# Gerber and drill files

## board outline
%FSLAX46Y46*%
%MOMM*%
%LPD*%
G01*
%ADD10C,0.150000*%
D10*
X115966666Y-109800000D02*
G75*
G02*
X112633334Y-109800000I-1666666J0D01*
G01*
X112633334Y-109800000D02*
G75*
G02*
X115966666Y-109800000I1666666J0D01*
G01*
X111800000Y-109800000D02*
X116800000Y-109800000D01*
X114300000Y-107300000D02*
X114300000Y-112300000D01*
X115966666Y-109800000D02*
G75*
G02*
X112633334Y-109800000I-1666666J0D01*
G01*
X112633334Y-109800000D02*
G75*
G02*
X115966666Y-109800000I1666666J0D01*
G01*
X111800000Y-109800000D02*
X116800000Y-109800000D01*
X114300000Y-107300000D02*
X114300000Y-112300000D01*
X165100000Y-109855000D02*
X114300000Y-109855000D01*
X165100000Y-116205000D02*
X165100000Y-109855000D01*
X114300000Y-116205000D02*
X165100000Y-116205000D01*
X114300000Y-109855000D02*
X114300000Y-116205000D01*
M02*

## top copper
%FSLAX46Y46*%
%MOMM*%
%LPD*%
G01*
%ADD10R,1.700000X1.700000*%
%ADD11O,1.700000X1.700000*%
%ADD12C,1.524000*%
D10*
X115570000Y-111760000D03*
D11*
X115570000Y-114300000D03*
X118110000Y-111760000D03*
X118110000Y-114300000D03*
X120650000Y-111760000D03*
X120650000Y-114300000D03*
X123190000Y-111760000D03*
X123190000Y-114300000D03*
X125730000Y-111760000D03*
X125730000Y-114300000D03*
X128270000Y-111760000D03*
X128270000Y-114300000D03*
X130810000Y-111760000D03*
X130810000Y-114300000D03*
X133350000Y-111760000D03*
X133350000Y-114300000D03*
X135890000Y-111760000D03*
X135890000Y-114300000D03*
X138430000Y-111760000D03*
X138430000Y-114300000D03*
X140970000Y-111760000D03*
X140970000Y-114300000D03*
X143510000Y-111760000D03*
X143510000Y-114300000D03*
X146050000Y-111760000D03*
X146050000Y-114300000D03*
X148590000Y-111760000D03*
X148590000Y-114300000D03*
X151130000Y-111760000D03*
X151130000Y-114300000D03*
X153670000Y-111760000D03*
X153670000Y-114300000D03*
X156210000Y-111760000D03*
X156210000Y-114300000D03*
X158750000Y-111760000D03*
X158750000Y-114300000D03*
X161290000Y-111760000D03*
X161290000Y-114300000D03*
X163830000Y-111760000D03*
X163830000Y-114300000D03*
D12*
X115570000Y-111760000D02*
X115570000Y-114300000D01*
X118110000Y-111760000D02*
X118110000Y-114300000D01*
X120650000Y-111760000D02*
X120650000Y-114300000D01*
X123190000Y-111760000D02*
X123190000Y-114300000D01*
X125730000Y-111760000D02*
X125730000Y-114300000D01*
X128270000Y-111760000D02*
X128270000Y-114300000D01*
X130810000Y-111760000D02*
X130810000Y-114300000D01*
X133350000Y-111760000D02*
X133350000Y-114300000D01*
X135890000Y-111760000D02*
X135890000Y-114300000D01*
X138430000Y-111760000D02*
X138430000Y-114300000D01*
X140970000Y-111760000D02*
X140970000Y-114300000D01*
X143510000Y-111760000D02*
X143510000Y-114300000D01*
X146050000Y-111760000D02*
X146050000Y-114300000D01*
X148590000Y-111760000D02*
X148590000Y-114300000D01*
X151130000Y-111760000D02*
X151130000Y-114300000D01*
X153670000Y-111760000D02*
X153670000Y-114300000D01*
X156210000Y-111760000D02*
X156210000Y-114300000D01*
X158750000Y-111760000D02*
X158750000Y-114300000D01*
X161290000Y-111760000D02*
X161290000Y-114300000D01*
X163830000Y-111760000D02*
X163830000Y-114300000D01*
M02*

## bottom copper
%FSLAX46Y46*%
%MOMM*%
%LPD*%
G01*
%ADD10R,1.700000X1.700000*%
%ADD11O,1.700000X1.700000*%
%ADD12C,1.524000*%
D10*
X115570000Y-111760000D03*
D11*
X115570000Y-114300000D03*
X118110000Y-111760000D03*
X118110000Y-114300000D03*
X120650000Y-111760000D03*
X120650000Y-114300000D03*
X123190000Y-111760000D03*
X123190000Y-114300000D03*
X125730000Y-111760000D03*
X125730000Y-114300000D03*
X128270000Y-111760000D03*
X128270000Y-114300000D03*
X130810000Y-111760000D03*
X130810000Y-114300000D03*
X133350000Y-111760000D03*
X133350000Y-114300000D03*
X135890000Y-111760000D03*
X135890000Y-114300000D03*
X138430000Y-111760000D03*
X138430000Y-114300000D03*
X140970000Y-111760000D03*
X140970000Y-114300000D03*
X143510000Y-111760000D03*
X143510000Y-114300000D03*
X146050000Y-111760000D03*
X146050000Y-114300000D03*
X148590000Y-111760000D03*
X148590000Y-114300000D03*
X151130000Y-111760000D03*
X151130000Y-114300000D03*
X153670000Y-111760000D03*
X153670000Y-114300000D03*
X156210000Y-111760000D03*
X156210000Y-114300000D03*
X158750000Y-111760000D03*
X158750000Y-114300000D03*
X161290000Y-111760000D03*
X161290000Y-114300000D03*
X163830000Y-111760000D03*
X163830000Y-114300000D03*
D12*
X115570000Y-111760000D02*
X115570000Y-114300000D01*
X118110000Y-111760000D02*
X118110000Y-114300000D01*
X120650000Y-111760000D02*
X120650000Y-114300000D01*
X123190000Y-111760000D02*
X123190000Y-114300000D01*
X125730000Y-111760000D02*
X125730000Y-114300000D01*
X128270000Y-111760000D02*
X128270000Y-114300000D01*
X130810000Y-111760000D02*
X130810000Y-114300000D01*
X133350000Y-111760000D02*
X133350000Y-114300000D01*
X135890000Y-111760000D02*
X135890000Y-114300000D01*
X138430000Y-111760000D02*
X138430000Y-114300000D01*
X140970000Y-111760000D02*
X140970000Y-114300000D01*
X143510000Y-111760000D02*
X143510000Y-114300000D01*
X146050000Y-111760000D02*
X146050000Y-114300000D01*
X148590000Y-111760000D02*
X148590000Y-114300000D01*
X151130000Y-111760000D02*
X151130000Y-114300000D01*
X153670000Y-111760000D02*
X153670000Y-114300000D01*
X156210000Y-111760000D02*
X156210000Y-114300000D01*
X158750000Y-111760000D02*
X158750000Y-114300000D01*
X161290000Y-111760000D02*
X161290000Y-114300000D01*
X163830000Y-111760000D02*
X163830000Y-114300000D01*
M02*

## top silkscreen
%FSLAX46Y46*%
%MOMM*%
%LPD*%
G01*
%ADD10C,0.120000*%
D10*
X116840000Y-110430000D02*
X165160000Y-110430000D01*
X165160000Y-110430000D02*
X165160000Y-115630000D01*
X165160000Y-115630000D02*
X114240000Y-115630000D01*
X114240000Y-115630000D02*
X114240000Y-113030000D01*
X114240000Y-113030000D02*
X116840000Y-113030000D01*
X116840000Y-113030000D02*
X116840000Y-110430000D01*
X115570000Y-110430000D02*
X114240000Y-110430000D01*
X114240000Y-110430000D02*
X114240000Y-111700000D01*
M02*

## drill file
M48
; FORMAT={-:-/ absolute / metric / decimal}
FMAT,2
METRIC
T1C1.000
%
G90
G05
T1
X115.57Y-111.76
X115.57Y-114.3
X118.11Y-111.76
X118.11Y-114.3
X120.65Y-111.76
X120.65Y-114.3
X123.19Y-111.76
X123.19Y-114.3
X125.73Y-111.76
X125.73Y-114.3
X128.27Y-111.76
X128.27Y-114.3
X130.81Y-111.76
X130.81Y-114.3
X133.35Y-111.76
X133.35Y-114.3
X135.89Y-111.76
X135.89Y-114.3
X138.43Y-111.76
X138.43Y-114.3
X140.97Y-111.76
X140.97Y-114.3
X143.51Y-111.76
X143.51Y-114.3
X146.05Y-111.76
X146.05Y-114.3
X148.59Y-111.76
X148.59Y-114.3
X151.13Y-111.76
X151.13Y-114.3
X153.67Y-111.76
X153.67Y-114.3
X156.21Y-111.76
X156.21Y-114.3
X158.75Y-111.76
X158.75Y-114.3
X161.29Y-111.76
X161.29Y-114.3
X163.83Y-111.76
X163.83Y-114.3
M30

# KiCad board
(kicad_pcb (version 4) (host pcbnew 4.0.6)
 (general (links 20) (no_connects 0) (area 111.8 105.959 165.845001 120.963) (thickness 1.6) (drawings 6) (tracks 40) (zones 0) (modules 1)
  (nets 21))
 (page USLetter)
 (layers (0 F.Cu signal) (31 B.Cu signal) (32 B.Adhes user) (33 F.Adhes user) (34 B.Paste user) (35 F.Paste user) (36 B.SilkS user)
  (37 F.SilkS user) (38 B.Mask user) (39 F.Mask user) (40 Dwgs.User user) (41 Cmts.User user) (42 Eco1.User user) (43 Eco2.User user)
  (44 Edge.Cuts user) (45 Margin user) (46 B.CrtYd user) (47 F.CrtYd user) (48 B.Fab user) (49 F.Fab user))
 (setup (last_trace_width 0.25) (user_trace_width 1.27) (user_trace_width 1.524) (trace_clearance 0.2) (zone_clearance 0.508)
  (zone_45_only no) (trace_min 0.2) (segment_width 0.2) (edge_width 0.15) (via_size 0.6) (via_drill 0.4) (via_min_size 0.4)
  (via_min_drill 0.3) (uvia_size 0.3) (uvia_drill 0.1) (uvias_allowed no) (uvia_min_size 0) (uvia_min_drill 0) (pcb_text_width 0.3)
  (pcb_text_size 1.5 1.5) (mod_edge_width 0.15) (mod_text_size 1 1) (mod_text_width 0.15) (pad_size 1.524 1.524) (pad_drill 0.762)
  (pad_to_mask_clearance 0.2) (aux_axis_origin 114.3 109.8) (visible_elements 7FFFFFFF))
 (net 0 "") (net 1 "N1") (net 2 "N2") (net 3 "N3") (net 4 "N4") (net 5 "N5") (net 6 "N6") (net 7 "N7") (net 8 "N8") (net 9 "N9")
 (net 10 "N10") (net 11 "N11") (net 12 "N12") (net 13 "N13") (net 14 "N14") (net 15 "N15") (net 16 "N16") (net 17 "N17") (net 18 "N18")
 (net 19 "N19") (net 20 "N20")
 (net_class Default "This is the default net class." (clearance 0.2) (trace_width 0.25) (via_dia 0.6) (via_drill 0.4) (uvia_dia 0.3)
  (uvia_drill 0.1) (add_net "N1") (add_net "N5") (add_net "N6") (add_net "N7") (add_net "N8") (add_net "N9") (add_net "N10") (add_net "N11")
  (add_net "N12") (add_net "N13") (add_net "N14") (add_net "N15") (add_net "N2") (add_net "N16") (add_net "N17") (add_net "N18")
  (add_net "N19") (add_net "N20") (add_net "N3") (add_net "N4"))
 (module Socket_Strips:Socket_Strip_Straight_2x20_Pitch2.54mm (layer F.Cu) (at 115.57 111.76 90)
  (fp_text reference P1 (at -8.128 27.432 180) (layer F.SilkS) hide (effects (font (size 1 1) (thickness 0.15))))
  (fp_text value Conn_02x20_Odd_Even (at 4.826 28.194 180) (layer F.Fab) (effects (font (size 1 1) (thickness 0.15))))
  (fp_line (start 1.33 1.27) (end 1.33 49.59) (layer F.SilkS) (width 0.12))
  (fp_line (start 1.33 49.59) (end -3.87 49.59) (layer F.SilkS) (width 0.12))
  (fp_line (start -3.87 49.59) (end -3.87 -1.33) (layer F.SilkS) (width 0.12))
  (fp_line (start -3.87 -1.33) (end -1.27 -1.33) (layer F.SilkS) (width 0.12))
  (fp_line (start -1.27 -1.33) (end -1.27 1.27) (layer F.SilkS) (width 0.12))
  (fp_line (start -1.27 1.27) (end 1.33 1.27) (layer F.SilkS) (width 0.12))
  (fp_line (start 1.33 0) (end 1.33 -1.33) (layer F.SilkS) (width 0.12))
  (fp_line (start 1.33 -1.33) (end 0.06 -1.33) (layer F.SilkS) (width 0.12))
  (pad 1 thru_hole rect (at 0 0 90) (size 1.7 1.7) (drill 1) (layers *.Cu *.Mask) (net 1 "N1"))
  (pad 2 thru_hole oval (at -2.54 0 90) (size 1.7 1.7) (drill 1) (layers *.Cu *.Mask) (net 1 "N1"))
  (pad 3 thru_hole oval (at 0 2.54 90) (size 1.7 1.7) (drill 1) (layers *.Cu *.Mask) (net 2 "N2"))
  (pad 4 thru_hole oval (at -2.54 2.54 90) (size 1.7 1.7) (drill 1) (layers *.Cu *.Mask) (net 2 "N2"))
  (pad 5 thru_hole oval (at 0 5.08 90) (size 1.7 1.7) (drill 1) (layers *.Cu *.Mask) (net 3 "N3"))
  (pad 6 thru_hole oval (at -2.54 5.08 90) (size 1.7 1.7) (drill 1) (layers *.Cu *.Mask) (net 3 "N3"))
  (pad 7 thru_hole oval (at 0 7.62 90) (size 1.7 1.7) (drill 1) (layers *.Cu *.Mask) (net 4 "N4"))
  (pad 8 thru_hole oval (at -2.54 7.62 90) (size 1.7 1.7) (drill 1) (layers *.Cu *.Mask) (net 4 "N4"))
  (pad 9 thru_hole oval (at 0 10.16 90) (size 1.7 1.7) (drill 1) (layers *.Cu *.Mask) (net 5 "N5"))
  (pad 10 thru_hole oval (at -2.54 10.16 90) (size 1.7 1.7) (drill 1) (layers *.Cu *.Mask) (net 5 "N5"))
  (pad 11 thru_hole oval (at 0 12.7 90) (size 1.7 1.7) (drill 1) (layers *.Cu *.Mask) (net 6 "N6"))
  (pad 12 thru_hole oval (at -2.54 12.7 90) (size 1.7 1.7) (drill 1) (layers *.Cu *.Mask) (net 6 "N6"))
  (pad 13 thru_hole oval (at 0 15.24 90) (size 1.7 1.7) (drill 1) (layers *.Cu *.Mask) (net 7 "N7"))
  (pad 14 thru_hole oval (at -2.54 15.24 90) (size 1.7 1.7) (drill 1) (layers *.Cu *.Mask) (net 7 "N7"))
  (pad 15 thru_hole oval (at 0 17.78 90) (size 1.7 1.7) (drill 1) (layers *.Cu *.Mask) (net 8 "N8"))
  (pad 16 thru_hole oval (at -2.54 17.78 90) (size 1.7 1.7) (drill 1) (layers *.Cu *.Mask) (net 8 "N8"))
  (pad 17 thru_hole oval (at 0 20.32 90) (size 1.7 1.7) (drill 1) (layers *.Cu *.Mask) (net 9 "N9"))
  (pad 18 thru_hole oval (at -2.54 20.32 90) (size 1.7 1.7) (drill 1) (layers *.Cu *.Mask) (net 9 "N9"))
  (pad 19 thru_hole oval (at 0 22.86 90) (size 1.7 1.7) (drill 1) (layers *.Cu *.Mask) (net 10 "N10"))
  (pad 20 thru_hole oval (at -2.54 22.86 90) (size 1.7 1.7) (drill 1) (layers *.Cu *.Mask) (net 10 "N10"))
  (pad 21 thru_hole oval (at 0 25.4 90) (size 1.7 1.7) (drill 1) (layers *.Cu *.Mask) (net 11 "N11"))
  (pad 22 thru_hole oval (at -2.54 25.4 90) (size 1.7 1.7) (drill 1) (layers *.Cu *.Mask) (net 11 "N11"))
  (pad 23 thru_hole oval (at 0 27.94 90) (size 1.7 1.7) (drill 1) (layers *.Cu *.Mask) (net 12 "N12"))
  (pad 24 thru_hole oval (at -2.54 27.94 90) (size 1.7 1.7) (drill 1) (layers *.Cu *.Mask) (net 12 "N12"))
  (pad 25 thru_hole oval (at 0 30.48 90) (size 1.7 1.7) (drill 1) (layers *.Cu *.Mask) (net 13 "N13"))
  (pad 26 thru_hole oval (at -2.54 30.48 90) (size 1.7 1.7) (drill 1) (layers *.Cu *.Mask) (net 13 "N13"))
  (pad 27 thru_hole oval (at 0 33.02 90) (size 1.7 1.7) (drill 1) (layers *.Cu *.Mask) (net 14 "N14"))
  (pad 28 thru_hole oval (at -2.54 33.02 90) (size 1.7 1.7) (drill 1) (layers *.Cu *.Mask) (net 14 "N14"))
  (pad 29 thru_hole oval (at 0 35.56 90) (size 1.7 1.7) (drill 1) (layers *.Cu *.Mask) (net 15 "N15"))
  (pad 30 thru_hole oval (at -2.54 35.56 90) (size 1.7 1.7) (drill 1) (layers *.Cu *.Mask) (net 15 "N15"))
  (pad 31 thru_hole oval (at 0 38.1 90) (size 1.7 1.7) (drill 1) (layers *.Cu *.Mask) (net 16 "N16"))
  (pad 32 thru_hole oval (at -2.54 38.1 90) (size 1.7 1.7) (drill 1) (layers *.Cu *.Mask) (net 16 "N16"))
  (pad 33 thru_hole oval (at 0 40.64 90) (size 1.7 1.7) (drill 1) (layers *.Cu *.Mask) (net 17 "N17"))
  (pad 34 thru_hole oval (at -2.54 40.64 90) (size 1.7 1.7) (drill 1) (layers *.Cu *.Mask) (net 17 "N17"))
  (pad 35 thru_hole oval (at 0 43.18 90) (size 1.7 1.7) (drill 1) (layers *.Cu *.Mask) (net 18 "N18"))
  (pad 36 thru_hole oval (at -2.54 43.18 90) (size 1.7 1.7) (drill 1) (layers *.Cu *.Mask) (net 18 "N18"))
  (pad 37 thru_hole oval (at 0 45.72 90) (size 1.7 1.7) (drill 1) (layers *.Cu *.Mask) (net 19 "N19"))
  (pad 38 thru_hole oval (at -2.54 45.72 90) (size 1.7 1.7) (drill 1) (layers *.Cu *.Mask) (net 19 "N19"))
  (pad 39 thru_hole oval (at 0 48.26 90) (size 1.7 1.7) (drill 1) (layers *.Cu *.Mask) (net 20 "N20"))
  (pad 40 thru_hole oval (at -2.54 48.26 90) (size 1.7 1.7) (drill 1) (layers *.Cu *.Mask) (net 20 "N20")))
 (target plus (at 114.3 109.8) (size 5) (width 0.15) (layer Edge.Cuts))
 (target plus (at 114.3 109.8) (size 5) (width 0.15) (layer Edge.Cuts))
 (gr_line (start 165.1 109.855) (end 114.3 109.855) (angle 90) (layer Edge.Cuts) (width 0.15))
 (gr_line (start 165.1 116.205) (end 165.1 109.855) (angle 90) (layer Edge.Cuts) (width 0.15))
 (gr_line (start 114.3 116.205) (end 165.1 116.205) (angle 90) (layer Edge.Cuts) (width 0.15))
 (gr_line (start 114.3 109.855) (end 114.3 116.205) (angle 90) (layer Edge.Cuts) (width 0.15))
 (segment (start 115.57 111.76) (end 115.57 114.3) (width 1.524) (layer F.Cu) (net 1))
 (segment (start 115.57 111.76) (end 115.57 114.3) (width 1.524) (layer B.Cu) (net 1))
 (segment (start 118.11 111.76) (end 118.11 114.3) (width 1.524) (layer B.Cu) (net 2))
 (segment (start 118.11 111.76) (end 118.11 114.3) (width 1.524) (layer F.Cu) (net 2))
 (segment (start 120.65 111.76) (end 120.65 114.3) (width 1.524) (layer B.Cu) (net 3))
 (segment (start 120.65 111.76) (end 120.65 114.3) (width 1.524) (layer F.Cu) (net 3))
 (segment (start 123.19 111.76) (end 123.19 114.3) (width 1.524) (layer B.Cu) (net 4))
 (segment (start 123.19 111.76) (end 123.19 114.3) (width 1.524) (layer F.Cu) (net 4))
 (segment (start 125.73 111.76) (end 125.73 114.3) (width 1.524) (layer B.Cu) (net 5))
 (segment (start 125.73 111.76) (end 125.73 114.3) (width 1.524) (layer F.Cu) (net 5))
 (segment (start 128.27 111.76) (end 128.27 114.3) (width 1.524) (layer B.Cu) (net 6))
 (segment (start 128.27 111.76) (end 128.27 114.3) (width 1.524) (layer F.Cu) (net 6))
 (segment (start 130.81 111.76) (end 130.81 114.3) (width 1.524) (layer B.Cu) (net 7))
 (segment (start 130.81 111.76) (end 130.81 114.3) (width 1.524) (layer F.Cu) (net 7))
 (segment (start 133.35 111.76) (end 133.35 114.3) (width 1.524) (layer B.Cu) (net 8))
 (segment (start 133.35 111.76) (end 133.35 114.3) (width 1.524) (layer F.Cu) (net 8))
 (segment (start 135.89 111.76) (end 135.89 114.3) (width 1.524) (layer B.Cu) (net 9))
 (segment (start 135.89 111.76) (end 135.89 114.3) (width 1.524) (layer F.Cu) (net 9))
 (segment (start 138.43 111.76) (end 138.43 114.3) (width 1.524) (layer B.Cu) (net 10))
 (segment (start 138.43 111.76) (end 138.43 114.3) (width 1.524) (layer F.Cu) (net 10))
 (segment (start 140.97 111.76) (end 140.97 114.3) (width 1.524) (layer B.Cu) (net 11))
 (segment (start 140.97 111.76) (end 140.97 114.3) (width 1.524) (layer F.Cu) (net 11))
 (segment (start 143.51 111.76) (end 143.51 114.3) (width 1.524) (layer B.Cu) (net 12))
 (segment (start 143.51 111.76) (end 143.51 114.3) (width 1.524) (layer F.Cu) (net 12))
 (segment (start 146.05 111.76) (end 146.05 114.3) (width 1.524) (layer B.Cu) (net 13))
 (segment (start 146.05 111.76) (end 146.05 114.3) (width 1.524) (layer F.Cu) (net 13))
 (segment (start 148.59 111.76) (end 148.59 114.3) (width 1.524) (layer B.Cu) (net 14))
 (segment (start 148.59 111.76) (end 148.59 114.3) (width 1.524) (layer F.Cu) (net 14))
 (segment (start 151.13 111.76) (end 151.13 114.3) (width 1.524) (layer B.Cu) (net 15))
 (segment (start 151.13 111.76) (end 151.13 114.3) (width 1.524) (layer F.Cu) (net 15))
 (segment (start 153.67 111.76) (end 153.67 114.3) (width 1.524) (layer B.Cu) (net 16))
 (segment (start 153.67 111.76) (end 153.67 114.3) (width 1.524) (layer F.Cu) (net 16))
 (segment (start 156.21 111.76) (end 156.21 114.3) (width 1.524) (layer B.Cu) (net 17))
 (segment (start 156.21 111.76) (end 156.21 114.3) (width 1.524) (layer F.Cu) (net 17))
 (segment (start 158.75 111.76) (end 158.75 114.3) (width 1.524) (layer B.Cu) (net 18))
 (segment (start 158.75 111.76) (end 158.75 114.3) (width 1.524) (layer F.Cu) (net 18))
 (segment (start 161.29 111.76) (end 161.29 114.3) (width 1.524) (layer B.Cu) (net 19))
 (segment (start 161.29 111.76) (end 161.29 114.3) (width 1.524) (layer F.Cu) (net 19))
 (segment (start 163.83 111.76) (end 163.83 114.3) (width 1.524) (layer B.Cu) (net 20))
 (segment (start 163.83 111.76) (end 163.83 114.3) (width 1.524) (layer F.Cu) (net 20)))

